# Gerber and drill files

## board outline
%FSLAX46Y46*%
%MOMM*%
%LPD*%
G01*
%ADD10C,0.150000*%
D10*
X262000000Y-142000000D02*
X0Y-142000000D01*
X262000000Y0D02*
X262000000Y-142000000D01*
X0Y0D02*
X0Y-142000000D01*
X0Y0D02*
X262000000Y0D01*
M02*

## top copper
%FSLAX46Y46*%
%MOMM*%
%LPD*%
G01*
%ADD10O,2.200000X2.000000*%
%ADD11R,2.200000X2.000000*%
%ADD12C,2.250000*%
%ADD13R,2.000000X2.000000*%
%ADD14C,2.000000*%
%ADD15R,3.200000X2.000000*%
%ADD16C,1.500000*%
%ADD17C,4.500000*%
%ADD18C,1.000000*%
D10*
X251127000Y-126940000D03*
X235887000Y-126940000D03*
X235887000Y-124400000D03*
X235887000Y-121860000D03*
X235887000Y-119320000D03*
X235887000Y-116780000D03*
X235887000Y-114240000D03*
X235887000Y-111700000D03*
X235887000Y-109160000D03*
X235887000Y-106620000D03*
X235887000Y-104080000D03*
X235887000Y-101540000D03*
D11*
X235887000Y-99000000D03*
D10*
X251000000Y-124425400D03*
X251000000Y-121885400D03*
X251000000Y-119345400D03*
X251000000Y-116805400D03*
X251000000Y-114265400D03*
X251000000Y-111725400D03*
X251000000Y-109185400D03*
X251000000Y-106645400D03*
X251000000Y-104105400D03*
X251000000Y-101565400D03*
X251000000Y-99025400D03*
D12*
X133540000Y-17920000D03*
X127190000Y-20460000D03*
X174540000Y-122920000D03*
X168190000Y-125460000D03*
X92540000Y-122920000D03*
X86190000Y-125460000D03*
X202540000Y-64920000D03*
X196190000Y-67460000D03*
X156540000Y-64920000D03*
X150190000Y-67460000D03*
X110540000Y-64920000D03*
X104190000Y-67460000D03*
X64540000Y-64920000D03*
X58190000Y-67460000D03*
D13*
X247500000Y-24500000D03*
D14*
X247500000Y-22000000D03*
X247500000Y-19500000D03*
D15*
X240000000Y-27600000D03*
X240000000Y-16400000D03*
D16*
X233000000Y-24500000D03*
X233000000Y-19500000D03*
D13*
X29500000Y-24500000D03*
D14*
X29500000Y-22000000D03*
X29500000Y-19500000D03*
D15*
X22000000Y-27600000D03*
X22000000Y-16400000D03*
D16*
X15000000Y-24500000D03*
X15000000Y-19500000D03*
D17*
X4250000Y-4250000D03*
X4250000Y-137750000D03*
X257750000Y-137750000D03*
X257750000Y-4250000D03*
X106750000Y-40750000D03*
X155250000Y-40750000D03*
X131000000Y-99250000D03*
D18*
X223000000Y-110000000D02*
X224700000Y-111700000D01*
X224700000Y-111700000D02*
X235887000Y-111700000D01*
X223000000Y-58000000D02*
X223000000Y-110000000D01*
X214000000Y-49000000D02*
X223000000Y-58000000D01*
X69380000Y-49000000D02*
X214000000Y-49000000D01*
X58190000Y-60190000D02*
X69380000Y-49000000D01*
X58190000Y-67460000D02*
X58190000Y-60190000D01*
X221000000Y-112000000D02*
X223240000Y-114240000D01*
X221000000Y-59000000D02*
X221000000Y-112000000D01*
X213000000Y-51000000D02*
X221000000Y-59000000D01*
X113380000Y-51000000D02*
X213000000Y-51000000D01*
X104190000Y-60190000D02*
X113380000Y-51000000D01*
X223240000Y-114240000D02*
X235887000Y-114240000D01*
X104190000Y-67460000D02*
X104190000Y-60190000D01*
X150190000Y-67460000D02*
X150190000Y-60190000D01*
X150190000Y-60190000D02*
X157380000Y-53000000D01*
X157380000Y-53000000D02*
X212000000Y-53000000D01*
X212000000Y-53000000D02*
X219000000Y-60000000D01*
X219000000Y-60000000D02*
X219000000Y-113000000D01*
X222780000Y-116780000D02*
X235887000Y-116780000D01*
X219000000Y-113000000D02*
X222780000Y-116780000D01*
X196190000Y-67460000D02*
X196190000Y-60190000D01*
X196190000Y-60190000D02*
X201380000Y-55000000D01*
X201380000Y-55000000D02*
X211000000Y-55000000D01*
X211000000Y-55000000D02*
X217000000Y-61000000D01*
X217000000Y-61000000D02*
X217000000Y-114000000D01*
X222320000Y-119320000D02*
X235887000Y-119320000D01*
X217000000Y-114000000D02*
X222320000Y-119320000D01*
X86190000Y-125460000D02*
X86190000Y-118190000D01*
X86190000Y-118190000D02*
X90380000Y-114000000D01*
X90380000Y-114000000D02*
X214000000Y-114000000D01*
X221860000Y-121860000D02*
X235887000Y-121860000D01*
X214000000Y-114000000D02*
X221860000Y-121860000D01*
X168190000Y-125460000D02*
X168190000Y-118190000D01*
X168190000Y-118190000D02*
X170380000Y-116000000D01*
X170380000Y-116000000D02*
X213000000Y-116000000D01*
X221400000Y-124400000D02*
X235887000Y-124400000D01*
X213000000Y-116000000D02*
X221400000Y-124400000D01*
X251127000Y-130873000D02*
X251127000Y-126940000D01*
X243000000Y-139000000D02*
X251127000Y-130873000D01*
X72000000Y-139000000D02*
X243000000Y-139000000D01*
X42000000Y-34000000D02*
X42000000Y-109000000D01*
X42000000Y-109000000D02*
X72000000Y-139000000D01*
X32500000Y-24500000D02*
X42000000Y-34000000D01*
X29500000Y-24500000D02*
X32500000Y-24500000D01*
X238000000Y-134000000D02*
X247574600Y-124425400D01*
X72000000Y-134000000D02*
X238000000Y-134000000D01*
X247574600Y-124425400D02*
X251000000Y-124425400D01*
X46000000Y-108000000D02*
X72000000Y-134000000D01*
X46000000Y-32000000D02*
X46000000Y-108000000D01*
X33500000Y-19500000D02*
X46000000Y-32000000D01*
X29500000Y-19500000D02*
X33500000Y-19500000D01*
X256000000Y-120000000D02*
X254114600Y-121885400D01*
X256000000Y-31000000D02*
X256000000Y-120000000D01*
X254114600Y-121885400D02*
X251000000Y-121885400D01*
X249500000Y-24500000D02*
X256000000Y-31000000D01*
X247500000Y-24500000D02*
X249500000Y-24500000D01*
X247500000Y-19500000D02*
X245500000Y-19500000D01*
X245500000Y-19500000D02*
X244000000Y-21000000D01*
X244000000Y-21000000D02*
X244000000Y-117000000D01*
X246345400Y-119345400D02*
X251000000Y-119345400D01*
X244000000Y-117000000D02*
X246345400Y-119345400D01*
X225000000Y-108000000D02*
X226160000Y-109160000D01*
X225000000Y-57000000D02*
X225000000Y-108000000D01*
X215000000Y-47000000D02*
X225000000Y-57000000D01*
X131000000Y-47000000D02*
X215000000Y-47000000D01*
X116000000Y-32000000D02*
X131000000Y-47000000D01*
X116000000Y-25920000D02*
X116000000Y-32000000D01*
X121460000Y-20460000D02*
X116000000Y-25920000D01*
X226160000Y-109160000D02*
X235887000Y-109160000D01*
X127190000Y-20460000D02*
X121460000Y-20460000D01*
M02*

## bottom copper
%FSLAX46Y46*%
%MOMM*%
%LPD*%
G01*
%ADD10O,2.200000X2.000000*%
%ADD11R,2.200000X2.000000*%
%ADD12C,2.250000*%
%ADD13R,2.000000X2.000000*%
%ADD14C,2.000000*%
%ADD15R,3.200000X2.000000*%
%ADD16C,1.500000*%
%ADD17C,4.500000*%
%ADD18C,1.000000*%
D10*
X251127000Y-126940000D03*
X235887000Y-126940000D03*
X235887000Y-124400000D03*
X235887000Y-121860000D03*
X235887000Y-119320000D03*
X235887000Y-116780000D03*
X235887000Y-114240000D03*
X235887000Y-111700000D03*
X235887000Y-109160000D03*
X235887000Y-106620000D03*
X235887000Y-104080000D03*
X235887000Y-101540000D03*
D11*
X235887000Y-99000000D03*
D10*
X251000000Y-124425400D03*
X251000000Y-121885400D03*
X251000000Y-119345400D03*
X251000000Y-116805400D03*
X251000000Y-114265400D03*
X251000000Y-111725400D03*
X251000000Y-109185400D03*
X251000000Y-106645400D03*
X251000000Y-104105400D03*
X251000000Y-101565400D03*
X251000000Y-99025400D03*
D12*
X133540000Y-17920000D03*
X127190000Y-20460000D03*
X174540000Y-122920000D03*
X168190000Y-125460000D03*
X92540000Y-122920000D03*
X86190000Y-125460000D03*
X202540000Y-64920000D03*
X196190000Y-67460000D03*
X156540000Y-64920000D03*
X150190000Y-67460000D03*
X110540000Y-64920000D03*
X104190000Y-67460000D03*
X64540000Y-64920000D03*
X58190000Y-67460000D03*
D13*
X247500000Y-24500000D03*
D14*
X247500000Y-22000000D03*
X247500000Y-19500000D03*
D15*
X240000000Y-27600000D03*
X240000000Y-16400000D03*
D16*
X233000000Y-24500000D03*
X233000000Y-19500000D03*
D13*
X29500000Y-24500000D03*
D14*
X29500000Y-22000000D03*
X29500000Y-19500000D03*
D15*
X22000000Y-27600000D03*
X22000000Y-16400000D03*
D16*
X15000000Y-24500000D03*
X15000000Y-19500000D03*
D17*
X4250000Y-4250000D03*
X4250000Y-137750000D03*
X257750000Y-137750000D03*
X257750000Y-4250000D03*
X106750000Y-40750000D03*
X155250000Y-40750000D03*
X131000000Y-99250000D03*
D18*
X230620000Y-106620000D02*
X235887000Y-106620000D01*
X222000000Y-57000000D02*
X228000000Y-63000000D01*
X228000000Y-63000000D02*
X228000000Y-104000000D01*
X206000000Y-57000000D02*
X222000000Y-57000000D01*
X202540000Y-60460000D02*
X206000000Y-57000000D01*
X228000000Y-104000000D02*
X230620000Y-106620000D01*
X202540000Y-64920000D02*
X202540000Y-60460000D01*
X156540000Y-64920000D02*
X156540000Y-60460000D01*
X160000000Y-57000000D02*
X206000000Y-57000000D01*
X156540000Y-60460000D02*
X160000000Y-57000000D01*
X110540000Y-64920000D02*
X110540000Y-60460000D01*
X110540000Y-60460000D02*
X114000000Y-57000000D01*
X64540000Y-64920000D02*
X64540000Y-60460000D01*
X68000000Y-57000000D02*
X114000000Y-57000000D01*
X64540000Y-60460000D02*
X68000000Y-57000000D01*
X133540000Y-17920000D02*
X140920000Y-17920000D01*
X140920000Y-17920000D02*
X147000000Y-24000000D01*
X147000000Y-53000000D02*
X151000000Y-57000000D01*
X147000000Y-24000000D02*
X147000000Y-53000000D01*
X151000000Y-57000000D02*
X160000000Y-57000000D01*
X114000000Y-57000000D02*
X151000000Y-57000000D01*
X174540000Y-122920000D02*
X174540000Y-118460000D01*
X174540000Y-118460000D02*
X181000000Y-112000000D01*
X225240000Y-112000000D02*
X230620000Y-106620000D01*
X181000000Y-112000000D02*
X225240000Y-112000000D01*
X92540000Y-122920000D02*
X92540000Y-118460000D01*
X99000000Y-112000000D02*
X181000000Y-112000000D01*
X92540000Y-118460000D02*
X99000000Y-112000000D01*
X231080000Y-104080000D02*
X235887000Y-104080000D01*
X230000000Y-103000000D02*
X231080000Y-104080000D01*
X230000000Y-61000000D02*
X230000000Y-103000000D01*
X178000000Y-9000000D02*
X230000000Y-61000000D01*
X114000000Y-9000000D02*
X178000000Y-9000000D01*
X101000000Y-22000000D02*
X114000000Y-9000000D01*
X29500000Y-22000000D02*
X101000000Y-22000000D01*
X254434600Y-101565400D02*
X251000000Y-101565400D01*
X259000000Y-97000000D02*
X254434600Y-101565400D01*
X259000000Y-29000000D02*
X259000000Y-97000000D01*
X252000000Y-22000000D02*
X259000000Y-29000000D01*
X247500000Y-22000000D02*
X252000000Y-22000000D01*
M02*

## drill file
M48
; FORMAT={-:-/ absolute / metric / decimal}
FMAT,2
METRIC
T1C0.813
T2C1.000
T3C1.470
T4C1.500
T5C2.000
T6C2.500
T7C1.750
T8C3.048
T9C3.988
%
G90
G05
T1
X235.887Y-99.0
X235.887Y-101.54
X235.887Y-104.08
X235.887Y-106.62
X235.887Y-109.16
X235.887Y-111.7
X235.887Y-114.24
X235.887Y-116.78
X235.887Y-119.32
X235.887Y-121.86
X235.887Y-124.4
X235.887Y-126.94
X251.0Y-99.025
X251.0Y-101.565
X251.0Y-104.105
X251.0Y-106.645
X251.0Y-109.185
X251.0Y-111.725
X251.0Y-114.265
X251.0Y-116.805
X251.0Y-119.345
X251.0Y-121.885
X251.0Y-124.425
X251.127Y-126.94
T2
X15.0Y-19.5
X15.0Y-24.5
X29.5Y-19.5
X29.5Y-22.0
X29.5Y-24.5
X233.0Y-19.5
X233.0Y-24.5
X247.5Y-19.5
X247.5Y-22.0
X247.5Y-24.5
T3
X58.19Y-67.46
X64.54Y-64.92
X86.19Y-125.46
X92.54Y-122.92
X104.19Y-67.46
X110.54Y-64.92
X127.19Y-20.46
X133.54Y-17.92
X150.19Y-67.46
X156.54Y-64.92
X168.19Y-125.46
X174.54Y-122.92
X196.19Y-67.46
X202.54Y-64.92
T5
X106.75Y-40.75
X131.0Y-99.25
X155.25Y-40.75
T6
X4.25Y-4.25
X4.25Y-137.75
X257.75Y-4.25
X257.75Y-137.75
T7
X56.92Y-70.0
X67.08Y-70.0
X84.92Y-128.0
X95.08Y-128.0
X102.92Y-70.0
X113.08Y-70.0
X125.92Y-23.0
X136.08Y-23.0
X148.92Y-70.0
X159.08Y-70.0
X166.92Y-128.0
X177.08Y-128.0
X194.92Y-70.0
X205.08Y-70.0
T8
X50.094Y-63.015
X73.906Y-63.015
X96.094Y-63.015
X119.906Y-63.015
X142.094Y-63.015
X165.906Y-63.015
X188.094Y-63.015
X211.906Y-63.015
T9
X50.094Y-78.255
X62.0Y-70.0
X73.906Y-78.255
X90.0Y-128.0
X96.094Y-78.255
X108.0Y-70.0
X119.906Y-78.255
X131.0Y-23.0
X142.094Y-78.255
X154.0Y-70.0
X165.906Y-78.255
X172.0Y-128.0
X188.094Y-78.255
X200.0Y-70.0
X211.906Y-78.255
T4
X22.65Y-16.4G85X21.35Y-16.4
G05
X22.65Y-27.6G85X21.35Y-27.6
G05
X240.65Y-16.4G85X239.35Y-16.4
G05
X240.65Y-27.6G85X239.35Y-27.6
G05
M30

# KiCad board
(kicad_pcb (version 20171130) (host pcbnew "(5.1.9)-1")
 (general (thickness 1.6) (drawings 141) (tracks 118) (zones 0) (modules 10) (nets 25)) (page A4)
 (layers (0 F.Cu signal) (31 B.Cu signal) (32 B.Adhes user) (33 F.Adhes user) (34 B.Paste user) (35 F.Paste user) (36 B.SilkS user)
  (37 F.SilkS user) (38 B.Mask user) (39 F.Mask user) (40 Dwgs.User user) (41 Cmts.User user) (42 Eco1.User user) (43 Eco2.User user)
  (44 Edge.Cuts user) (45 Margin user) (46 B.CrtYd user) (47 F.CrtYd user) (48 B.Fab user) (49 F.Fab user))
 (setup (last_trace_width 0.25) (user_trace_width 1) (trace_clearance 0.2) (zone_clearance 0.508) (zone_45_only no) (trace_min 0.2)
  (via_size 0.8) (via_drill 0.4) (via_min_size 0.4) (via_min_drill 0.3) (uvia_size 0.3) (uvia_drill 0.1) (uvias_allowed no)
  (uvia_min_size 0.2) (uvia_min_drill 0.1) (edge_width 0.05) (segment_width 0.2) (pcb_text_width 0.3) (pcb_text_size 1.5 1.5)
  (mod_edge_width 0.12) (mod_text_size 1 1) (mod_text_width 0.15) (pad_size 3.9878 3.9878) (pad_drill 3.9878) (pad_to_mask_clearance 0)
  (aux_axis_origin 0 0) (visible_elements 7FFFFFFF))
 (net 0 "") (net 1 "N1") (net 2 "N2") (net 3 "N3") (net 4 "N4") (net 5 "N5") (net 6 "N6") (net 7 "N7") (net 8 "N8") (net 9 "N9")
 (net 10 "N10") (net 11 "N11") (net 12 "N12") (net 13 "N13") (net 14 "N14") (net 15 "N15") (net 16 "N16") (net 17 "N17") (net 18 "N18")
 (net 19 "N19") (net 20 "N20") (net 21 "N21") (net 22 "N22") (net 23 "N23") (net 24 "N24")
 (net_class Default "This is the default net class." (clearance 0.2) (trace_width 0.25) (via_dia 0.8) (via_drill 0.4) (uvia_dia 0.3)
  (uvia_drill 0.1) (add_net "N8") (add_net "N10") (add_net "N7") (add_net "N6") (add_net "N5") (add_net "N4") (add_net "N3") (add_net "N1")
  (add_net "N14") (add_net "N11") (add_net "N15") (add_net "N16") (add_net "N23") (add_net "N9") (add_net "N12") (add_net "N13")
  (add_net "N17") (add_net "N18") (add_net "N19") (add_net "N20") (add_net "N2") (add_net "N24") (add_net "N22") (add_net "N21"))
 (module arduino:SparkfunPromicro (layer F.Cu) (at 235.887 99)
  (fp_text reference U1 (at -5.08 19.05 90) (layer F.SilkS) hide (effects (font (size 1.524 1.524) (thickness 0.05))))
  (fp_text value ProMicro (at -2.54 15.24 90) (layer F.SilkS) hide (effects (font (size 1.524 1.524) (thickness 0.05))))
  (pad 10 thru_hole oval (at 15.24 27.94) (size 2.2 2) (drill 0.8128) (layers *.Cu) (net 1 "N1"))
  (pad 9 thru_hole oval (at 0 27.94) (size 2.2 2) (drill 0.8128) (layers *.Cu) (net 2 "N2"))
  (pad 8 thru_hole oval (at 0 25.4) (size 2.2 2) (drill 0.8128) (layers *.Cu) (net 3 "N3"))
  (pad 7 thru_hole oval (at 0 22.86) (size 2.2 2) (drill 0.8128) (layers *.Cu) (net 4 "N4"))
  (pad 6 thru_hole oval (at 0 20.32) (size 2.2 2) (drill 0.8128) (layers *.Cu) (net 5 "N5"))
  (pad 5 thru_hole oval (at 0 17.78) (size 2.2 2) (drill 0.8128) (layers *.Cu) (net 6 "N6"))
  (pad 4 thru_hole oval (at 0 15.24) (size 2.2 2) (drill 0.8128) (layers *.Cu) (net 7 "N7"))
  (pad 3 thru_hole oval (at 0 12.7) (size 2.2 2) (drill 0.8128) (layers *.Cu) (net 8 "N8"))
  (pad 2 thru_hole oval (at 0 10.16) (size 2.2 2) (drill 0.8128) (layers *.Cu) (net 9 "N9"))
  (pad GND2 thru_hole oval (at 0 7.62) (size 2.2 2) (drill 0.8128) (layers *.Cu) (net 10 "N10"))
  (pad GND1 thru_hole oval (at 0 5.08) (size 2.2 2) (drill 0.8128) (layers *.Cu) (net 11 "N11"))
  (pad 0 thru_hole oval (at 0 2.54) (size 2.2 2) (drill 0.8128) (layers *.Cu) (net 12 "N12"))
  (pad 1 thru_hole rect (at 0 0) (size 2.2 2) (drill 0.8128) (layers *.Cu) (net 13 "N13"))
  (pad 16 thru_hole oval (at 15.113 25.4254) (size 2.2 2) (drill 0.8128) (layers *.Cu) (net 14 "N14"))
  (pad 14 thru_hole oval (at 15.113 22.8854) (size 2.2 2) (drill 0.8128) (layers *.Cu) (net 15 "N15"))
  (pad 15 thru_hole oval (at 15.113 20.3454) (size 2.2 2) (drill 0.8128) (layers *.Cu) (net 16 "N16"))
  (pad 18 thru_hole oval (at 15.113 17.8054) (size 2.2 2) (drill 0.8128) (layers *.Cu) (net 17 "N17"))
  (pad 19 thru_hole oval (at 15.113 15.2654) (size 2.2 2) (drill 0.8128) (layers *.Cu) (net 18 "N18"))
  (pad 20 thru_hole oval (at 15.113 12.7254) (size 2.2 2) (drill 0.8128) (layers *.Cu) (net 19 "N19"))
  (pad 21 thru_hole oval (at 15.113 10.1854) (size 2.2 2) (drill 0.8128) (layers *.Cu) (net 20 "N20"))
  (pad VCC thru_hole oval (at 15.113 7.6454) (size 2.2 2) (drill 0.8128) (layers *.Cu) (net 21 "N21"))
  (pad RST thru_hole oval (at 15.113 5.1054) (size 2.2 2) (drill 0.8128) (layers *.Cu) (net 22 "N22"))
  (pad GND3 thru_hole oval (at 15.113 2.5654) (size 2.2 2) (drill 0.8128) (layers *.Cu) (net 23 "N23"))
  (pad RAW thru_hole oval (at 15.113 0.0254) (size 2.2 2) (drill 0.8128) (layers *.Cu) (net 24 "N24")))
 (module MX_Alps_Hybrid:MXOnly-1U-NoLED (layer F.Cu) (at 131 23)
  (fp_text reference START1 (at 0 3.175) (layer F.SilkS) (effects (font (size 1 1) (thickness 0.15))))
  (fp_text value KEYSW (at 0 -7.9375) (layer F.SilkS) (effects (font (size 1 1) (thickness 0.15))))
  (pad 2 thru_hole circle (at 2.54 -5.08) (size 2.25 2.25) (drill 1.47) (layers *.Cu B.Mask) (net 10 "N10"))
  (pad "" np_thru_hole circle (at 0 0) (size 3.9878 3.9878) (drill 3.9878) (layers *.Cu *.Mask))
  (pad 1 thru_hole circle (at -3.81 -2.54) (size 2.25 2.25) (drill 1.47) (layers *.Cu B.Mask) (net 9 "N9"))
  (pad "" np_thru_hole circle (at -5.08 0 48.0996) (size 1.75 1.75) (drill 1.75) (layers *.Cu *.Mask))
  (pad "" np_thru_hole circle (at 5.08 0 48.0996) (size 1.75 1.75) (drill 1.75) (layers *.Cu *.Mask)))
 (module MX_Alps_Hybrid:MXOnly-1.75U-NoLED (layer F.Cu) (at 172 128)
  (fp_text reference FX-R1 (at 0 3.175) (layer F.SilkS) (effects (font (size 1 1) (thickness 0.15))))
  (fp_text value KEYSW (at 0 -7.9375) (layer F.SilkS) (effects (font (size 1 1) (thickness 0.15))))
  (pad 2 thru_hole circle (at 2.54 -5.08) (size 2.25 2.25) (drill 1.47) (layers *.Cu B.Mask) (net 10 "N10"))
  (pad "" np_thru_hole circle (at 0 0) (size 3.9878 3.9878) (drill 3.9878) (layers *.Cu *.Mask))
  (pad 1 thru_hole circle (at -3.81 -2.54) (size 2.25 2.25) (drill 1.47) (layers *.Cu B.Mask) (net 3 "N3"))
  (pad "" np_thru_hole circle (at -5.08 0 48.0996) (size 1.75 1.75) (drill 1.75) (layers *.Cu *.Mask))
  (pad "" np_thru_hole circle (at 5.08 0 48.0996) (size 1.75 1.75) (drill 1.75) (layers *.Cu *.Mask)))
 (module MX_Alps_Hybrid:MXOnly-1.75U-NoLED (layer F.Cu) (at 90 128)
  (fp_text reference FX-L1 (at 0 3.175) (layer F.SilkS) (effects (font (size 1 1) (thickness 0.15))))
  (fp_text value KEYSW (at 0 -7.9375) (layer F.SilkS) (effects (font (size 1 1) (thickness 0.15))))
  (pad 2 thru_hole circle (at 2.54 -5.08) (size 2.25 2.25) (drill 1.47) (layers *.Cu B.Mask) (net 10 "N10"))
  (pad "" np_thru_hole circle (at 0 0) (size 3.9878 3.9878) (drill 3.9878) (layers *.Cu *.Mask))
  (pad 1 thru_hole circle (at -3.81 -2.54) (size 2.25 2.25) (drill 1.47) (layers *.Cu B.Mask) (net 4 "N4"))
  (pad "" np_thru_hole circle (at -5.08 0 48.0996) (size 1.75 1.75) (drill 1.75) (layers *.Cu *.Mask))
  (pad "" np_thru_hole circle (at 5.08 0 48.0996) (size 1.75 1.75) (drill 1.75) (layers *.Cu *.Mask)))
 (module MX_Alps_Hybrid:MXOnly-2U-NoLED (layer F.Cu) (at 200 70)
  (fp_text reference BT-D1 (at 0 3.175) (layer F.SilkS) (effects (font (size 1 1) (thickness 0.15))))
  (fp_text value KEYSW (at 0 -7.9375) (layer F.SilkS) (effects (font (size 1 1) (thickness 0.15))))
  (pad 2 thru_hole circle (at 2.54 -5.08) (size 2.25 2.25) (drill 1.47) (layers *.Cu B.Mask) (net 10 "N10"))
  (pad "" np_thru_hole circle (at 0 0) (size 3.9878 3.9878) (drill 3.9878) (layers *.Cu *.Mask))
  (pad 1 thru_hole circle (at -3.81 -2.54) (size 2.25 2.25) (drill 1.47) (layers *.Cu B.Mask) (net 5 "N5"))
  (pad "" np_thru_hole circle (at -5.08 0 48.0996) (size 1.75 1.75) (drill 1.75) (layers *.Cu *.Mask))
  (pad "" np_thru_hole circle (at 5.08 0 48.0996) (size 1.75 1.75) (drill 1.75) (layers *.Cu *.Mask))
  (pad "" np_thru_hole circle (at -11.90625 -6.985) (size 3.048 3.048) (drill 3.048) (layers *.Cu *.Mask))
  (pad "" np_thru_hole circle (at 11.90625 -6.985) (size 3.048 3.048) (drill 3.048) (layers *.Cu *.Mask))
  (pad "" np_thru_hole circle (at -11.90625 8.255) (size 3.9878 3.9878) (drill 3.9878) (layers *.Cu *.Mask))
  (pad "" np_thru_hole circle (at 11.90625 8.255) (size 3.9878 3.9878) (drill 3.9878) (layers *.Cu *.Mask)))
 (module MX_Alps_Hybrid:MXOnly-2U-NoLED (layer F.Cu) (at 154 70)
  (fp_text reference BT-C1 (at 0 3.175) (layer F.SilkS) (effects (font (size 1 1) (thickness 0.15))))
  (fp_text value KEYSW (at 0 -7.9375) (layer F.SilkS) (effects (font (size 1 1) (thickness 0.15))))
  (pad 2 thru_hole circle (at 2.54 -5.08) (size 2.25 2.25) (drill 1.47) (layers *.Cu B.Mask) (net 10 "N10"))
  (pad "" np_thru_hole circle (at 0 0) (size 3.9878 3.9878) (drill 3.9878) (layers *.Cu *.Mask))
  (pad 1 thru_hole circle (at -3.81 -2.54) (size 2.25 2.25) (drill 1.47) (layers *.Cu B.Mask) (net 6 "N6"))
  (pad "" np_thru_hole circle (at -5.08 0 48.0996) (size 1.75 1.75) (drill 1.75) (layers *.Cu *.Mask))
  (pad "" np_thru_hole circle (at 5.08 0 48.0996) (size 1.75 1.75) (drill 1.75) (layers *.Cu *.Mask))
  (pad "" np_thru_hole circle (at -11.90625 -6.985) (size 3.048 3.048) (drill 3.048) (layers *.Cu *.Mask))
  (pad "" np_thru_hole circle (at 11.90625 -6.985) (size 3.048 3.048) (drill 3.048) (layers *.Cu *.Mask))
  (pad "" np_thru_hole circle (at -11.90625 8.255) (size 3.9878 3.9878) (drill 3.9878) (layers *.Cu *.Mask))
  (pad "" np_thru_hole circle (at 11.90625 8.255) (size 3.9878 3.9878) (drill 3.9878) (layers *.Cu *.Mask)))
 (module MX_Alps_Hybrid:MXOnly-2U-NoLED (layer F.Cu) (at 108 70)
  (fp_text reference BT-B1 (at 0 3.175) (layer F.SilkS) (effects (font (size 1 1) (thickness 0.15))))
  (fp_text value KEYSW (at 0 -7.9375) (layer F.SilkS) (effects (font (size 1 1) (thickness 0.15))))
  (pad 2 thru_hole circle (at 2.54 -5.08) (size 2.25 2.25) (drill 1.47) (layers *.Cu B.Mask) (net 10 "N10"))
  (pad "" np_thru_hole circle (at 0 0) (size 3.9878 3.9878) (drill 3.9878) (layers *.Cu *.Mask))
  (pad 1 thru_hole circle (at -3.81 -2.54) (size 2.25 2.25) (drill 1.47) (layers *.Cu B.Mask) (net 7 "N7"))
  (pad "" np_thru_hole circle (at -5.08 0 48.0996) (size 1.75 1.75) (drill 1.75) (layers *.Cu *.Mask))
  (pad "" np_thru_hole circle (at 5.08 0 48.0996) (size 1.75 1.75) (drill 1.75) (layers *.Cu *.Mask))
  (pad "" np_thru_hole circle (at -11.90625 -6.985) (size 3.048 3.048) (drill 3.048) (layers *.Cu *.Mask))
  (pad "" np_thru_hole circle (at 11.90625 -6.985) (size 3.048 3.048) (drill 3.048) (layers *.Cu *.Mask))
  (pad "" np_thru_hole circle (at -11.90625 8.255) (size 3.9878 3.9878) (drill 3.9878) (layers *.Cu *.Mask))
  (pad "" np_thru_hole circle (at 11.90625 8.255) (size 3.9878 3.9878) (drill 3.9878) (layers *.Cu *.Mask)))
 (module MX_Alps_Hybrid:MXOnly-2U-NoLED (layer F.Cu) (at 62 70)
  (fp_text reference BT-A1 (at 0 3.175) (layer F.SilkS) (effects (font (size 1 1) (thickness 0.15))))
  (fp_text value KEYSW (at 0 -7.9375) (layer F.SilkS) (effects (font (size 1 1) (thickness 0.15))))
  (pad 2 thru_hole circle (at 2.54 -5.08) (size 2.25 2.25) (drill 1.47) (layers *.Cu B.Mask) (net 10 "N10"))
  (pad "" np_thru_hole circle (at 0 0) (size 3.9878 3.9878) (drill 3.9878) (layers *.Cu *.Mask))
  (pad 1 thru_hole circle (at -3.81 -2.54) (size 2.25 2.25) (drill 1.47) (layers *.Cu B.Mask) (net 8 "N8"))
  (pad "" np_thru_hole circle (at -5.08 0 48.0996) (size 1.75 1.75) (drill 1.75) (layers *.Cu *.Mask))
  (pad "" np_thru_hole circle (at 5.08 0 48.0996) (size 1.75 1.75) (drill 1.75) (layers *.Cu *.Mask))
  (pad "" np_thru_hole circle (at -11.90625 -6.985) (size 3.048 3.048) (drill 3.048) (layers *.Cu *.Mask))
  (pad "" np_thru_hole circle (at 11.90625 -6.985) (size 3.048 3.048) (drill 3.048) (layers *.Cu *.Mask))
  (pad "" np_thru_hole circle (at -11.90625 8.255) (size 3.9878 3.9878) (drill 3.9878) (layers *.Cu *.Mask))
  (pad "" np_thru_hole circle (at 11.90625 8.255) (size 3.9878 3.9878) (drill 3.9878) (layers *.Cu *.Mask)))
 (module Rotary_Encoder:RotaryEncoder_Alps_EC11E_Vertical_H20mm (layer F.Cu) (at 247.5 24.5 180)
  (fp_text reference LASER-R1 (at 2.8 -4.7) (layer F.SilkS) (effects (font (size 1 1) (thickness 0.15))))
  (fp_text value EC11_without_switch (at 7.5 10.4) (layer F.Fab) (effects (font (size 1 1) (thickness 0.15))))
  (pad A thru_hole rect (at 0 0 180) (size 2 2) (drill 1) (layers *.Cu *.Mask) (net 15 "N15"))
  (pad C thru_hole circle (at 0 2.5 180) (size 2 2) (drill 1) (layers *.Cu *.Mask) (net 23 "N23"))
  (pad B thru_hole circle (at 0 5 180) (size 2 2) (drill 1) (layers *.Cu *.Mask) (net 16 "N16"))
  (pad MP thru_hole rect (at 7.5 -3.1 180) (size 3.2 2) (drill oval 2.8 1.5) (layers *.Cu *.Mask))
  (pad MP thru_hole rect (at 7.5 8.1 180) (size 3.2 2) (drill oval 2.8 1.5) (layers *.Cu *.Mask))
  (pad "" thru_hole circle (at 14.5 0 180) (size 1.5 1.5) (drill 1) (layers *.Cu *.Mask))
  (pad "" thru_hole circle (at 14.5 5 180) (size 1.5 1.5) (drill 1) (layers *.Cu *.Mask)))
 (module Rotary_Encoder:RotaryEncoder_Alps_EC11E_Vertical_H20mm (layer F.Cu) (at 29.5 24.5 180)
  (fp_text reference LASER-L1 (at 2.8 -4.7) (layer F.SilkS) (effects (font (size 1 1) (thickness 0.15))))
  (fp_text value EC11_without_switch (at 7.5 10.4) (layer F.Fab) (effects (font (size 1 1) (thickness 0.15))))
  (pad A thru_hole rect (at 0 0 180) (size 2 2) (drill 1) (layers *.Cu *.Mask) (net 1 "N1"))
  (pad C thru_hole circle (at 0 2.5 180) (size 2 2) (drill 1) (layers *.Cu *.Mask) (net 11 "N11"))
  (pad B thru_hole circle (at 0 5 180) (size 2 2) (drill 1) (layers *.Cu *.Mask) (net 14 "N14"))
  (pad MP thru_hole rect (at 7.5 -3.1 180) (size 3.2 2) (drill oval 2.8 1.5) (layers *.Cu *.Mask))
  (pad MP thru_hole rect (at 7.5 8.1 180) (size 3.2 2) (drill oval 2.8 1.5) (layers *.Cu *.Mask))
  (pad "" thru_hole circle (at 14.5 0 180) (size 1.5 1.5) (drill 1) (layers *.Cu *.Mask))
  (pad "" thru_hole circle (at 14.5 5 180) (size 1.5 1.5) (drill 1) (layers *.Cu *.Mask)))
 (gr_line (start 262 142) (end 0 142) (layer Edge.Cuts) (width 0.15))
 (gr_line (start 262 0) (end 262 142) (layer Edge.Cuts) (width 0.15))
 (gr_line (start 0 0) (end 0 142) (layer Edge.Cuts) (width 0.15))
 (gr_line (start 0 0) (end 262 0) (layer Edge.Cuts) (width 0.15))
 (via (at 4.25 4.25) (size 4.5) (drill 2.5) (layers F.Cu B.Cu) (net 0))
 (via (at 4.25 137.75) (size 4.5) (drill 2.5) (layers F.Cu B.Cu) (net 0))
 (via (at 257.75 137.75) (size 4.5) (drill 2.5) (layers F.Cu B.Cu) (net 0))
 (via (at 257.75 4.25) (size 4.5) (drill 2.5) (layers F.Cu B.Cu) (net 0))
 (via (at 106.75 40.75) (size 4.5) (drill 2) (layers F.Cu B.Cu) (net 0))
 (via (at 155.25 40.75) (size 4.5) (drill 2) (layers F.Cu B.Cu) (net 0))
 (via (at 131 99.25) (size 4.5) (drill 2) (layers F.Cu B.Cu) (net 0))
 (segment (start 223 110) (end 224.7 111.7) (width 1) (layer F.Cu) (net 8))
 (segment (start 224.7 111.7) (end 235.887 111.7) (width 1) (layer F.Cu) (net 8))
 (segment (start 223 58) (end 223 110) (width 1) (layer F.Cu) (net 8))
 (segment (start 214 49) (end 223 58) (width 1) (layer F.Cu) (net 8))
 (segment (start 69.38 49) (end 214 49) (width 1) (layer F.Cu) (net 8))
 (segment (start 58.19 60.19) (end 69.38 49) (width 1) (layer F.Cu) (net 8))
 (segment (start 58.19 67.46) (end 58.19 60.19) (width 1) (layer F.Cu) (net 8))
 (segment (start 230.62 106.62) (end 235.887 106.62) (width 1) (layer B.Cu) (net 10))
 (segment (start 222 57) (end 228 63) (width 1) (layer B.Cu) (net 10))
 (segment (start 228 63) (end 228 104) (width 1) (layer B.Cu) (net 10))
 (segment (start 206 57) (end 222 57) (width 1) (layer B.Cu) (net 10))
 (segment (start 202.54 60.46) (end 206 57) (width 1) (layer B.Cu) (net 10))
 (segment (start 228 104) (end 230.62 106.62) (width 1) (layer B.Cu) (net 10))
 (segment (start 202.54 64.92) (end 202.54 60.46) (width 1) (layer B.Cu) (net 10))
 (segment (start 156.54 64.92) (end 156.54 60.46) (width 1) (layer B.Cu) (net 10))
 (segment (start 160 57) (end 206 57) (width 1) (layer B.Cu) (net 10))
 (segment (start 156.54 60.46) (end 160 57) (width 1) (layer B.Cu) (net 10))
 (segment (start 110.54 64.92) (end 110.54 60.46) (width 1) (layer B.Cu) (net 10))
 (segment (start 110.54 60.46) (end 114 57) (width 1) (layer B.Cu) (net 10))
 (segment (start 64.54 64.92) (end 64.54 60.46) (width 1) (layer B.Cu) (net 10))
 (segment (start 68 57) (end 114 57) (width 1) (layer B.Cu) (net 10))
 (segment (start 64.54 60.46) (end 68 57) (width 1) (layer B.Cu) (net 10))
 (segment (start 133.54 17.92) (end 140.92 17.92) (width 1) (layer B.Cu) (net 10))
 (segment (start 140.92 17.92) (end 147 24) (width 1) (layer B.Cu) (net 10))
 (segment (start 147 53) (end 151 57) (width 1) (layer B.Cu) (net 10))
 (segment (start 147 24) (end 147 53) (width 1) (layer B.Cu) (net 10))
 (segment (start 151 57) (end 160 57) (width 1) (layer B.Cu) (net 10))
 (segment (start 114 57) (end 151 57) (width 1) (layer B.Cu) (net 10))
 (segment (start 174.54 122.92) (end 174.54 118.46) (width 1) (layer B.Cu) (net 10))
 (segment (start 174.54 118.46) (end 181 112) (width 1) (layer B.Cu) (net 10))
 (segment (start 225.24 112) (end 230.62 106.62) (width 1) (layer B.Cu) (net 10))
 (segment (start 181 112) (end 225.24 112) (width 1) (layer B.Cu) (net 10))
 (segment (start 92.54 122.92) (end 92.54 118.46) (width 1) (layer B.Cu) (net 10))
 (segment (start 99 112) (end 181 112) (width 1) (layer B.Cu) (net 10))
 (segment (start 92.54 118.46) (end 99 112) (width 1) (layer B.Cu) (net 10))
 (segment (start 221 112) (end 223.24 114.24) (width 1) (layer F.Cu) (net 7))
 (segment (start 221 59) (end 221 112) (width 1) (layer F.Cu) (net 7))
 (segment (start 213 51) (end 221 59) (width 1) (layer F.Cu) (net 7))
 (segment (start 113.38 51) (end 213 51) (width 1) (layer F.Cu) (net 7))
 (segment (start 104.19 60.19) (end 113.38 51) (width 1) (layer F.Cu) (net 7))
 (segment (start 223.24 114.24) (end 235.887 114.24) (width 1) (layer F.Cu) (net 7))
 (segment (start 104.19 67.46) (end 104.19 60.19) (width 1) (layer F.Cu) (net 7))
 (segment (start 150.19 67.46) (end 150.19 60.19) (width 1) (layer F.Cu) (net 6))
 (segment (start 150.19 60.19) (end 157.38 53) (width 1) (layer F.Cu) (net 6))
 (segment (start 157.38 53) (end 212 53) (width 1) (layer F.Cu) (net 6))
 (segment (start 212 53) (end 219 60) (width 1) (layer F.Cu) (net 6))
 (segment (start 219 60) (end 219 113) (width 1) (layer F.Cu) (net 6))
 (segment (start 222.78 116.78) (end 235.887 116.78) (width 1) (layer F.Cu) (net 6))
 (segment (start 219 113) (end 222.78 116.78) (width 1) (layer F.Cu) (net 6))
 (segment (start 196.19 67.46) (end 196.19 60.19) (width 1) (layer F.Cu) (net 5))
 (segment (start 196.19 60.19) (end 201.38 55) (width 1) (layer F.Cu) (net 5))
 (segment (start 201.38 55) (end 211 55) (width 1) (layer F.Cu) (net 5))
 (segment (start 211 55) (end 217 61) (width 1) (layer F.Cu) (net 5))
 (segment (start 217 61) (end 217 114) (width 1) (layer F.Cu) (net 5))
 (segment (start 222.32 119.32) (end 235.887 119.32) (width 1) (layer F.Cu) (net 5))
 (segment (start 217 114) (end 222.32 119.32) (width 1) (layer F.Cu) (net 5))
 (segment (start 86.19 125.46) (end 86.19 118.19) (width 1) (layer F.Cu) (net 4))
 (segment (start 86.19 118.19) (end 90.38 114) (width 1) (layer F.Cu) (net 4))
 (segment (start 90.38 114) (end 214 114) (width 1) (layer F.Cu) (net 4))
 (segment (start 221.86 121.86) (end 235.887 121.86) (width 1) (layer F.Cu) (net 4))
 (segment (start 214 114) (end 221.86 121.86) (width 1) (layer F.Cu) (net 4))
 (segment (start 168.19 125.46) (end 168.19 118.19) (width 1) (layer F.Cu) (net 3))
 (segment (start 168.19 118.19) (end 170.38 116) (width 1) (layer F.Cu) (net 3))
 (segment (start 170.38 116) (end 213 116) (width 1) (layer F.Cu) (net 3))
 (segment (start 221.4 124.4) (end 235.887 124.4) (width 1) (layer F.Cu) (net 3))
 (segment (start 213 116) (end 221.4 124.4) (width 1) (layer F.Cu) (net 3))
 (segment (start 251.127 130.873) (end 251.127 126.94) (width 1) (layer F.Cu) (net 1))
 (segment (start 243 139) (end 251.127 130.873) (width 1) (layer F.Cu) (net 1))
 (segment (start 72 139) (end 243 139) (width 1) (layer F.Cu) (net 1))
 (segment (start 42 34) (end 42 109) (width 1) (layer F.Cu) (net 1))
 (segment (start 42 109) (end 72 139) (width 1) (layer F.Cu) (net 1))
 (segment (start 32.5 24.5) (end 42 34) (width 1) (layer F.Cu) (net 1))
 (segment (start 29.5 24.5) (end 32.5 24.5) (width 1) (layer F.Cu) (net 1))
 (segment (start 231.08 104.08) (end 235.887 104.08) (width 1) (layer B.Cu) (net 11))
 (segment (start 230 103) (end 231.08 104.08) (width 1) (layer B.Cu) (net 11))
 (segment (start 230 61) (end 230 103) (width 1) (layer B.Cu) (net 11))
 (segment (start 178 9) (end 230 61) (width 1) (layer B.Cu) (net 11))
 (segment (start 114 9) (end 178 9) (width 1) (layer B.Cu) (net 11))
 (segment (start 101 22) (end 114 9) (width 1) (layer B.Cu) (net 11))
 (segment (start 29.5 22) (end 101 22) (width 1) (layer B.Cu) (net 11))
 (segment (start 238 134) (end 247.5746 124.4254) (width 1) (layer F.Cu) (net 14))
 (segment (start 72 134) (end 238 134) (width 1) (layer F.Cu) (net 14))
 (segment (start 247.5746 124.4254) (end 251 124.4254) (width 1) (layer F.Cu) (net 14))
 (segment (start 46 108) (end 72 134) (width 1) (layer F.Cu) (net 14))
 (segment (start 46 32) (end 46 108) (width 1) (layer F.Cu) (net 14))
 (segment (start 33.5 19.5) (end 46 32) (width 1) (layer F.Cu) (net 14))
 (segment (start 29.5 19.5) (end 33.5 19.5) (width 1) (layer F.Cu) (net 14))
 (segment (start 256 120) (end 254.1146 121.8854) (width 1) (layer F.Cu) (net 15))
 (segment (start 256 31) (end 256 120) (width 1) (layer F.Cu) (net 15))
 (segment (start 254.1146 121.8854) (end 251 121.8854) (width 1) (layer F.Cu) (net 15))
 (segment (start 249.5 24.5) (end 256 31) (width 1) (layer F.Cu) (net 15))
 (segment (start 247.5 24.5) (end 249.5 24.5) (width 1) (layer F.Cu) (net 15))
 (segment (start 254.4346 101.5654) (end 251 101.5654) (width 1) (layer B.Cu) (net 23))
 (segment (start 259 97) (end 254.4346 101.5654) (width 1) (layer B.Cu) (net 23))
 (segment (start 259 29) (end 259 97) (width 1) (layer B.Cu) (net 23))
 (segment (start 252 22) (end 259 29) (width 1) (layer B.Cu) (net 23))
 (segment (start 247.5 22) (end 252 22) (width 1) (layer B.Cu) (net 23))
 (segment (start 247.5 19.5) (end 245.5 19.5) (width 1) (layer F.Cu) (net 16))
 (segment (start 245.5 19.5) (end 244 21) (width 1) (layer F.Cu) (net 16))
 (segment (start 244 21) (end 244 117) (width 1) (layer F.Cu) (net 16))
 (segment (start 246.3454 119.3454) (end 251 119.3454) (width 1) (layer F.Cu) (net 16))
 (segment (start 244 117) (end 246.3454 119.3454) (width 1) (layer F.Cu) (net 16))
 (segment (start 225 108) (end 226.16 109.16) (width 1) (layer F.Cu) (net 9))
 (segment (start 225 57) (end 225 108) (width 1) (layer F.Cu) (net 9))
 (segment (start 215 47) (end 225 57) (width 1) (layer F.Cu) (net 9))
 (segment (start 131 47) (end 215 47) (width 1) (layer F.Cu) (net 9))
 (segment (start 116 32) (end 131 47) (width 1) (layer F.Cu) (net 9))
 (segment (start 116 25.92) (end 116 32) (width 1) (layer F.Cu) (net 9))
 (segment (start 121.46 20.46) (end 116 25.92) (width 1) (layer F.Cu) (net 9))
 (segment (start 226.16 109.16) (end 235.887 109.16) (width 1) (layer F.Cu) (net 9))
 (segment (start 127.19 20.46) (end 121.46 20.46) (width 1) (layer F.Cu) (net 9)))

